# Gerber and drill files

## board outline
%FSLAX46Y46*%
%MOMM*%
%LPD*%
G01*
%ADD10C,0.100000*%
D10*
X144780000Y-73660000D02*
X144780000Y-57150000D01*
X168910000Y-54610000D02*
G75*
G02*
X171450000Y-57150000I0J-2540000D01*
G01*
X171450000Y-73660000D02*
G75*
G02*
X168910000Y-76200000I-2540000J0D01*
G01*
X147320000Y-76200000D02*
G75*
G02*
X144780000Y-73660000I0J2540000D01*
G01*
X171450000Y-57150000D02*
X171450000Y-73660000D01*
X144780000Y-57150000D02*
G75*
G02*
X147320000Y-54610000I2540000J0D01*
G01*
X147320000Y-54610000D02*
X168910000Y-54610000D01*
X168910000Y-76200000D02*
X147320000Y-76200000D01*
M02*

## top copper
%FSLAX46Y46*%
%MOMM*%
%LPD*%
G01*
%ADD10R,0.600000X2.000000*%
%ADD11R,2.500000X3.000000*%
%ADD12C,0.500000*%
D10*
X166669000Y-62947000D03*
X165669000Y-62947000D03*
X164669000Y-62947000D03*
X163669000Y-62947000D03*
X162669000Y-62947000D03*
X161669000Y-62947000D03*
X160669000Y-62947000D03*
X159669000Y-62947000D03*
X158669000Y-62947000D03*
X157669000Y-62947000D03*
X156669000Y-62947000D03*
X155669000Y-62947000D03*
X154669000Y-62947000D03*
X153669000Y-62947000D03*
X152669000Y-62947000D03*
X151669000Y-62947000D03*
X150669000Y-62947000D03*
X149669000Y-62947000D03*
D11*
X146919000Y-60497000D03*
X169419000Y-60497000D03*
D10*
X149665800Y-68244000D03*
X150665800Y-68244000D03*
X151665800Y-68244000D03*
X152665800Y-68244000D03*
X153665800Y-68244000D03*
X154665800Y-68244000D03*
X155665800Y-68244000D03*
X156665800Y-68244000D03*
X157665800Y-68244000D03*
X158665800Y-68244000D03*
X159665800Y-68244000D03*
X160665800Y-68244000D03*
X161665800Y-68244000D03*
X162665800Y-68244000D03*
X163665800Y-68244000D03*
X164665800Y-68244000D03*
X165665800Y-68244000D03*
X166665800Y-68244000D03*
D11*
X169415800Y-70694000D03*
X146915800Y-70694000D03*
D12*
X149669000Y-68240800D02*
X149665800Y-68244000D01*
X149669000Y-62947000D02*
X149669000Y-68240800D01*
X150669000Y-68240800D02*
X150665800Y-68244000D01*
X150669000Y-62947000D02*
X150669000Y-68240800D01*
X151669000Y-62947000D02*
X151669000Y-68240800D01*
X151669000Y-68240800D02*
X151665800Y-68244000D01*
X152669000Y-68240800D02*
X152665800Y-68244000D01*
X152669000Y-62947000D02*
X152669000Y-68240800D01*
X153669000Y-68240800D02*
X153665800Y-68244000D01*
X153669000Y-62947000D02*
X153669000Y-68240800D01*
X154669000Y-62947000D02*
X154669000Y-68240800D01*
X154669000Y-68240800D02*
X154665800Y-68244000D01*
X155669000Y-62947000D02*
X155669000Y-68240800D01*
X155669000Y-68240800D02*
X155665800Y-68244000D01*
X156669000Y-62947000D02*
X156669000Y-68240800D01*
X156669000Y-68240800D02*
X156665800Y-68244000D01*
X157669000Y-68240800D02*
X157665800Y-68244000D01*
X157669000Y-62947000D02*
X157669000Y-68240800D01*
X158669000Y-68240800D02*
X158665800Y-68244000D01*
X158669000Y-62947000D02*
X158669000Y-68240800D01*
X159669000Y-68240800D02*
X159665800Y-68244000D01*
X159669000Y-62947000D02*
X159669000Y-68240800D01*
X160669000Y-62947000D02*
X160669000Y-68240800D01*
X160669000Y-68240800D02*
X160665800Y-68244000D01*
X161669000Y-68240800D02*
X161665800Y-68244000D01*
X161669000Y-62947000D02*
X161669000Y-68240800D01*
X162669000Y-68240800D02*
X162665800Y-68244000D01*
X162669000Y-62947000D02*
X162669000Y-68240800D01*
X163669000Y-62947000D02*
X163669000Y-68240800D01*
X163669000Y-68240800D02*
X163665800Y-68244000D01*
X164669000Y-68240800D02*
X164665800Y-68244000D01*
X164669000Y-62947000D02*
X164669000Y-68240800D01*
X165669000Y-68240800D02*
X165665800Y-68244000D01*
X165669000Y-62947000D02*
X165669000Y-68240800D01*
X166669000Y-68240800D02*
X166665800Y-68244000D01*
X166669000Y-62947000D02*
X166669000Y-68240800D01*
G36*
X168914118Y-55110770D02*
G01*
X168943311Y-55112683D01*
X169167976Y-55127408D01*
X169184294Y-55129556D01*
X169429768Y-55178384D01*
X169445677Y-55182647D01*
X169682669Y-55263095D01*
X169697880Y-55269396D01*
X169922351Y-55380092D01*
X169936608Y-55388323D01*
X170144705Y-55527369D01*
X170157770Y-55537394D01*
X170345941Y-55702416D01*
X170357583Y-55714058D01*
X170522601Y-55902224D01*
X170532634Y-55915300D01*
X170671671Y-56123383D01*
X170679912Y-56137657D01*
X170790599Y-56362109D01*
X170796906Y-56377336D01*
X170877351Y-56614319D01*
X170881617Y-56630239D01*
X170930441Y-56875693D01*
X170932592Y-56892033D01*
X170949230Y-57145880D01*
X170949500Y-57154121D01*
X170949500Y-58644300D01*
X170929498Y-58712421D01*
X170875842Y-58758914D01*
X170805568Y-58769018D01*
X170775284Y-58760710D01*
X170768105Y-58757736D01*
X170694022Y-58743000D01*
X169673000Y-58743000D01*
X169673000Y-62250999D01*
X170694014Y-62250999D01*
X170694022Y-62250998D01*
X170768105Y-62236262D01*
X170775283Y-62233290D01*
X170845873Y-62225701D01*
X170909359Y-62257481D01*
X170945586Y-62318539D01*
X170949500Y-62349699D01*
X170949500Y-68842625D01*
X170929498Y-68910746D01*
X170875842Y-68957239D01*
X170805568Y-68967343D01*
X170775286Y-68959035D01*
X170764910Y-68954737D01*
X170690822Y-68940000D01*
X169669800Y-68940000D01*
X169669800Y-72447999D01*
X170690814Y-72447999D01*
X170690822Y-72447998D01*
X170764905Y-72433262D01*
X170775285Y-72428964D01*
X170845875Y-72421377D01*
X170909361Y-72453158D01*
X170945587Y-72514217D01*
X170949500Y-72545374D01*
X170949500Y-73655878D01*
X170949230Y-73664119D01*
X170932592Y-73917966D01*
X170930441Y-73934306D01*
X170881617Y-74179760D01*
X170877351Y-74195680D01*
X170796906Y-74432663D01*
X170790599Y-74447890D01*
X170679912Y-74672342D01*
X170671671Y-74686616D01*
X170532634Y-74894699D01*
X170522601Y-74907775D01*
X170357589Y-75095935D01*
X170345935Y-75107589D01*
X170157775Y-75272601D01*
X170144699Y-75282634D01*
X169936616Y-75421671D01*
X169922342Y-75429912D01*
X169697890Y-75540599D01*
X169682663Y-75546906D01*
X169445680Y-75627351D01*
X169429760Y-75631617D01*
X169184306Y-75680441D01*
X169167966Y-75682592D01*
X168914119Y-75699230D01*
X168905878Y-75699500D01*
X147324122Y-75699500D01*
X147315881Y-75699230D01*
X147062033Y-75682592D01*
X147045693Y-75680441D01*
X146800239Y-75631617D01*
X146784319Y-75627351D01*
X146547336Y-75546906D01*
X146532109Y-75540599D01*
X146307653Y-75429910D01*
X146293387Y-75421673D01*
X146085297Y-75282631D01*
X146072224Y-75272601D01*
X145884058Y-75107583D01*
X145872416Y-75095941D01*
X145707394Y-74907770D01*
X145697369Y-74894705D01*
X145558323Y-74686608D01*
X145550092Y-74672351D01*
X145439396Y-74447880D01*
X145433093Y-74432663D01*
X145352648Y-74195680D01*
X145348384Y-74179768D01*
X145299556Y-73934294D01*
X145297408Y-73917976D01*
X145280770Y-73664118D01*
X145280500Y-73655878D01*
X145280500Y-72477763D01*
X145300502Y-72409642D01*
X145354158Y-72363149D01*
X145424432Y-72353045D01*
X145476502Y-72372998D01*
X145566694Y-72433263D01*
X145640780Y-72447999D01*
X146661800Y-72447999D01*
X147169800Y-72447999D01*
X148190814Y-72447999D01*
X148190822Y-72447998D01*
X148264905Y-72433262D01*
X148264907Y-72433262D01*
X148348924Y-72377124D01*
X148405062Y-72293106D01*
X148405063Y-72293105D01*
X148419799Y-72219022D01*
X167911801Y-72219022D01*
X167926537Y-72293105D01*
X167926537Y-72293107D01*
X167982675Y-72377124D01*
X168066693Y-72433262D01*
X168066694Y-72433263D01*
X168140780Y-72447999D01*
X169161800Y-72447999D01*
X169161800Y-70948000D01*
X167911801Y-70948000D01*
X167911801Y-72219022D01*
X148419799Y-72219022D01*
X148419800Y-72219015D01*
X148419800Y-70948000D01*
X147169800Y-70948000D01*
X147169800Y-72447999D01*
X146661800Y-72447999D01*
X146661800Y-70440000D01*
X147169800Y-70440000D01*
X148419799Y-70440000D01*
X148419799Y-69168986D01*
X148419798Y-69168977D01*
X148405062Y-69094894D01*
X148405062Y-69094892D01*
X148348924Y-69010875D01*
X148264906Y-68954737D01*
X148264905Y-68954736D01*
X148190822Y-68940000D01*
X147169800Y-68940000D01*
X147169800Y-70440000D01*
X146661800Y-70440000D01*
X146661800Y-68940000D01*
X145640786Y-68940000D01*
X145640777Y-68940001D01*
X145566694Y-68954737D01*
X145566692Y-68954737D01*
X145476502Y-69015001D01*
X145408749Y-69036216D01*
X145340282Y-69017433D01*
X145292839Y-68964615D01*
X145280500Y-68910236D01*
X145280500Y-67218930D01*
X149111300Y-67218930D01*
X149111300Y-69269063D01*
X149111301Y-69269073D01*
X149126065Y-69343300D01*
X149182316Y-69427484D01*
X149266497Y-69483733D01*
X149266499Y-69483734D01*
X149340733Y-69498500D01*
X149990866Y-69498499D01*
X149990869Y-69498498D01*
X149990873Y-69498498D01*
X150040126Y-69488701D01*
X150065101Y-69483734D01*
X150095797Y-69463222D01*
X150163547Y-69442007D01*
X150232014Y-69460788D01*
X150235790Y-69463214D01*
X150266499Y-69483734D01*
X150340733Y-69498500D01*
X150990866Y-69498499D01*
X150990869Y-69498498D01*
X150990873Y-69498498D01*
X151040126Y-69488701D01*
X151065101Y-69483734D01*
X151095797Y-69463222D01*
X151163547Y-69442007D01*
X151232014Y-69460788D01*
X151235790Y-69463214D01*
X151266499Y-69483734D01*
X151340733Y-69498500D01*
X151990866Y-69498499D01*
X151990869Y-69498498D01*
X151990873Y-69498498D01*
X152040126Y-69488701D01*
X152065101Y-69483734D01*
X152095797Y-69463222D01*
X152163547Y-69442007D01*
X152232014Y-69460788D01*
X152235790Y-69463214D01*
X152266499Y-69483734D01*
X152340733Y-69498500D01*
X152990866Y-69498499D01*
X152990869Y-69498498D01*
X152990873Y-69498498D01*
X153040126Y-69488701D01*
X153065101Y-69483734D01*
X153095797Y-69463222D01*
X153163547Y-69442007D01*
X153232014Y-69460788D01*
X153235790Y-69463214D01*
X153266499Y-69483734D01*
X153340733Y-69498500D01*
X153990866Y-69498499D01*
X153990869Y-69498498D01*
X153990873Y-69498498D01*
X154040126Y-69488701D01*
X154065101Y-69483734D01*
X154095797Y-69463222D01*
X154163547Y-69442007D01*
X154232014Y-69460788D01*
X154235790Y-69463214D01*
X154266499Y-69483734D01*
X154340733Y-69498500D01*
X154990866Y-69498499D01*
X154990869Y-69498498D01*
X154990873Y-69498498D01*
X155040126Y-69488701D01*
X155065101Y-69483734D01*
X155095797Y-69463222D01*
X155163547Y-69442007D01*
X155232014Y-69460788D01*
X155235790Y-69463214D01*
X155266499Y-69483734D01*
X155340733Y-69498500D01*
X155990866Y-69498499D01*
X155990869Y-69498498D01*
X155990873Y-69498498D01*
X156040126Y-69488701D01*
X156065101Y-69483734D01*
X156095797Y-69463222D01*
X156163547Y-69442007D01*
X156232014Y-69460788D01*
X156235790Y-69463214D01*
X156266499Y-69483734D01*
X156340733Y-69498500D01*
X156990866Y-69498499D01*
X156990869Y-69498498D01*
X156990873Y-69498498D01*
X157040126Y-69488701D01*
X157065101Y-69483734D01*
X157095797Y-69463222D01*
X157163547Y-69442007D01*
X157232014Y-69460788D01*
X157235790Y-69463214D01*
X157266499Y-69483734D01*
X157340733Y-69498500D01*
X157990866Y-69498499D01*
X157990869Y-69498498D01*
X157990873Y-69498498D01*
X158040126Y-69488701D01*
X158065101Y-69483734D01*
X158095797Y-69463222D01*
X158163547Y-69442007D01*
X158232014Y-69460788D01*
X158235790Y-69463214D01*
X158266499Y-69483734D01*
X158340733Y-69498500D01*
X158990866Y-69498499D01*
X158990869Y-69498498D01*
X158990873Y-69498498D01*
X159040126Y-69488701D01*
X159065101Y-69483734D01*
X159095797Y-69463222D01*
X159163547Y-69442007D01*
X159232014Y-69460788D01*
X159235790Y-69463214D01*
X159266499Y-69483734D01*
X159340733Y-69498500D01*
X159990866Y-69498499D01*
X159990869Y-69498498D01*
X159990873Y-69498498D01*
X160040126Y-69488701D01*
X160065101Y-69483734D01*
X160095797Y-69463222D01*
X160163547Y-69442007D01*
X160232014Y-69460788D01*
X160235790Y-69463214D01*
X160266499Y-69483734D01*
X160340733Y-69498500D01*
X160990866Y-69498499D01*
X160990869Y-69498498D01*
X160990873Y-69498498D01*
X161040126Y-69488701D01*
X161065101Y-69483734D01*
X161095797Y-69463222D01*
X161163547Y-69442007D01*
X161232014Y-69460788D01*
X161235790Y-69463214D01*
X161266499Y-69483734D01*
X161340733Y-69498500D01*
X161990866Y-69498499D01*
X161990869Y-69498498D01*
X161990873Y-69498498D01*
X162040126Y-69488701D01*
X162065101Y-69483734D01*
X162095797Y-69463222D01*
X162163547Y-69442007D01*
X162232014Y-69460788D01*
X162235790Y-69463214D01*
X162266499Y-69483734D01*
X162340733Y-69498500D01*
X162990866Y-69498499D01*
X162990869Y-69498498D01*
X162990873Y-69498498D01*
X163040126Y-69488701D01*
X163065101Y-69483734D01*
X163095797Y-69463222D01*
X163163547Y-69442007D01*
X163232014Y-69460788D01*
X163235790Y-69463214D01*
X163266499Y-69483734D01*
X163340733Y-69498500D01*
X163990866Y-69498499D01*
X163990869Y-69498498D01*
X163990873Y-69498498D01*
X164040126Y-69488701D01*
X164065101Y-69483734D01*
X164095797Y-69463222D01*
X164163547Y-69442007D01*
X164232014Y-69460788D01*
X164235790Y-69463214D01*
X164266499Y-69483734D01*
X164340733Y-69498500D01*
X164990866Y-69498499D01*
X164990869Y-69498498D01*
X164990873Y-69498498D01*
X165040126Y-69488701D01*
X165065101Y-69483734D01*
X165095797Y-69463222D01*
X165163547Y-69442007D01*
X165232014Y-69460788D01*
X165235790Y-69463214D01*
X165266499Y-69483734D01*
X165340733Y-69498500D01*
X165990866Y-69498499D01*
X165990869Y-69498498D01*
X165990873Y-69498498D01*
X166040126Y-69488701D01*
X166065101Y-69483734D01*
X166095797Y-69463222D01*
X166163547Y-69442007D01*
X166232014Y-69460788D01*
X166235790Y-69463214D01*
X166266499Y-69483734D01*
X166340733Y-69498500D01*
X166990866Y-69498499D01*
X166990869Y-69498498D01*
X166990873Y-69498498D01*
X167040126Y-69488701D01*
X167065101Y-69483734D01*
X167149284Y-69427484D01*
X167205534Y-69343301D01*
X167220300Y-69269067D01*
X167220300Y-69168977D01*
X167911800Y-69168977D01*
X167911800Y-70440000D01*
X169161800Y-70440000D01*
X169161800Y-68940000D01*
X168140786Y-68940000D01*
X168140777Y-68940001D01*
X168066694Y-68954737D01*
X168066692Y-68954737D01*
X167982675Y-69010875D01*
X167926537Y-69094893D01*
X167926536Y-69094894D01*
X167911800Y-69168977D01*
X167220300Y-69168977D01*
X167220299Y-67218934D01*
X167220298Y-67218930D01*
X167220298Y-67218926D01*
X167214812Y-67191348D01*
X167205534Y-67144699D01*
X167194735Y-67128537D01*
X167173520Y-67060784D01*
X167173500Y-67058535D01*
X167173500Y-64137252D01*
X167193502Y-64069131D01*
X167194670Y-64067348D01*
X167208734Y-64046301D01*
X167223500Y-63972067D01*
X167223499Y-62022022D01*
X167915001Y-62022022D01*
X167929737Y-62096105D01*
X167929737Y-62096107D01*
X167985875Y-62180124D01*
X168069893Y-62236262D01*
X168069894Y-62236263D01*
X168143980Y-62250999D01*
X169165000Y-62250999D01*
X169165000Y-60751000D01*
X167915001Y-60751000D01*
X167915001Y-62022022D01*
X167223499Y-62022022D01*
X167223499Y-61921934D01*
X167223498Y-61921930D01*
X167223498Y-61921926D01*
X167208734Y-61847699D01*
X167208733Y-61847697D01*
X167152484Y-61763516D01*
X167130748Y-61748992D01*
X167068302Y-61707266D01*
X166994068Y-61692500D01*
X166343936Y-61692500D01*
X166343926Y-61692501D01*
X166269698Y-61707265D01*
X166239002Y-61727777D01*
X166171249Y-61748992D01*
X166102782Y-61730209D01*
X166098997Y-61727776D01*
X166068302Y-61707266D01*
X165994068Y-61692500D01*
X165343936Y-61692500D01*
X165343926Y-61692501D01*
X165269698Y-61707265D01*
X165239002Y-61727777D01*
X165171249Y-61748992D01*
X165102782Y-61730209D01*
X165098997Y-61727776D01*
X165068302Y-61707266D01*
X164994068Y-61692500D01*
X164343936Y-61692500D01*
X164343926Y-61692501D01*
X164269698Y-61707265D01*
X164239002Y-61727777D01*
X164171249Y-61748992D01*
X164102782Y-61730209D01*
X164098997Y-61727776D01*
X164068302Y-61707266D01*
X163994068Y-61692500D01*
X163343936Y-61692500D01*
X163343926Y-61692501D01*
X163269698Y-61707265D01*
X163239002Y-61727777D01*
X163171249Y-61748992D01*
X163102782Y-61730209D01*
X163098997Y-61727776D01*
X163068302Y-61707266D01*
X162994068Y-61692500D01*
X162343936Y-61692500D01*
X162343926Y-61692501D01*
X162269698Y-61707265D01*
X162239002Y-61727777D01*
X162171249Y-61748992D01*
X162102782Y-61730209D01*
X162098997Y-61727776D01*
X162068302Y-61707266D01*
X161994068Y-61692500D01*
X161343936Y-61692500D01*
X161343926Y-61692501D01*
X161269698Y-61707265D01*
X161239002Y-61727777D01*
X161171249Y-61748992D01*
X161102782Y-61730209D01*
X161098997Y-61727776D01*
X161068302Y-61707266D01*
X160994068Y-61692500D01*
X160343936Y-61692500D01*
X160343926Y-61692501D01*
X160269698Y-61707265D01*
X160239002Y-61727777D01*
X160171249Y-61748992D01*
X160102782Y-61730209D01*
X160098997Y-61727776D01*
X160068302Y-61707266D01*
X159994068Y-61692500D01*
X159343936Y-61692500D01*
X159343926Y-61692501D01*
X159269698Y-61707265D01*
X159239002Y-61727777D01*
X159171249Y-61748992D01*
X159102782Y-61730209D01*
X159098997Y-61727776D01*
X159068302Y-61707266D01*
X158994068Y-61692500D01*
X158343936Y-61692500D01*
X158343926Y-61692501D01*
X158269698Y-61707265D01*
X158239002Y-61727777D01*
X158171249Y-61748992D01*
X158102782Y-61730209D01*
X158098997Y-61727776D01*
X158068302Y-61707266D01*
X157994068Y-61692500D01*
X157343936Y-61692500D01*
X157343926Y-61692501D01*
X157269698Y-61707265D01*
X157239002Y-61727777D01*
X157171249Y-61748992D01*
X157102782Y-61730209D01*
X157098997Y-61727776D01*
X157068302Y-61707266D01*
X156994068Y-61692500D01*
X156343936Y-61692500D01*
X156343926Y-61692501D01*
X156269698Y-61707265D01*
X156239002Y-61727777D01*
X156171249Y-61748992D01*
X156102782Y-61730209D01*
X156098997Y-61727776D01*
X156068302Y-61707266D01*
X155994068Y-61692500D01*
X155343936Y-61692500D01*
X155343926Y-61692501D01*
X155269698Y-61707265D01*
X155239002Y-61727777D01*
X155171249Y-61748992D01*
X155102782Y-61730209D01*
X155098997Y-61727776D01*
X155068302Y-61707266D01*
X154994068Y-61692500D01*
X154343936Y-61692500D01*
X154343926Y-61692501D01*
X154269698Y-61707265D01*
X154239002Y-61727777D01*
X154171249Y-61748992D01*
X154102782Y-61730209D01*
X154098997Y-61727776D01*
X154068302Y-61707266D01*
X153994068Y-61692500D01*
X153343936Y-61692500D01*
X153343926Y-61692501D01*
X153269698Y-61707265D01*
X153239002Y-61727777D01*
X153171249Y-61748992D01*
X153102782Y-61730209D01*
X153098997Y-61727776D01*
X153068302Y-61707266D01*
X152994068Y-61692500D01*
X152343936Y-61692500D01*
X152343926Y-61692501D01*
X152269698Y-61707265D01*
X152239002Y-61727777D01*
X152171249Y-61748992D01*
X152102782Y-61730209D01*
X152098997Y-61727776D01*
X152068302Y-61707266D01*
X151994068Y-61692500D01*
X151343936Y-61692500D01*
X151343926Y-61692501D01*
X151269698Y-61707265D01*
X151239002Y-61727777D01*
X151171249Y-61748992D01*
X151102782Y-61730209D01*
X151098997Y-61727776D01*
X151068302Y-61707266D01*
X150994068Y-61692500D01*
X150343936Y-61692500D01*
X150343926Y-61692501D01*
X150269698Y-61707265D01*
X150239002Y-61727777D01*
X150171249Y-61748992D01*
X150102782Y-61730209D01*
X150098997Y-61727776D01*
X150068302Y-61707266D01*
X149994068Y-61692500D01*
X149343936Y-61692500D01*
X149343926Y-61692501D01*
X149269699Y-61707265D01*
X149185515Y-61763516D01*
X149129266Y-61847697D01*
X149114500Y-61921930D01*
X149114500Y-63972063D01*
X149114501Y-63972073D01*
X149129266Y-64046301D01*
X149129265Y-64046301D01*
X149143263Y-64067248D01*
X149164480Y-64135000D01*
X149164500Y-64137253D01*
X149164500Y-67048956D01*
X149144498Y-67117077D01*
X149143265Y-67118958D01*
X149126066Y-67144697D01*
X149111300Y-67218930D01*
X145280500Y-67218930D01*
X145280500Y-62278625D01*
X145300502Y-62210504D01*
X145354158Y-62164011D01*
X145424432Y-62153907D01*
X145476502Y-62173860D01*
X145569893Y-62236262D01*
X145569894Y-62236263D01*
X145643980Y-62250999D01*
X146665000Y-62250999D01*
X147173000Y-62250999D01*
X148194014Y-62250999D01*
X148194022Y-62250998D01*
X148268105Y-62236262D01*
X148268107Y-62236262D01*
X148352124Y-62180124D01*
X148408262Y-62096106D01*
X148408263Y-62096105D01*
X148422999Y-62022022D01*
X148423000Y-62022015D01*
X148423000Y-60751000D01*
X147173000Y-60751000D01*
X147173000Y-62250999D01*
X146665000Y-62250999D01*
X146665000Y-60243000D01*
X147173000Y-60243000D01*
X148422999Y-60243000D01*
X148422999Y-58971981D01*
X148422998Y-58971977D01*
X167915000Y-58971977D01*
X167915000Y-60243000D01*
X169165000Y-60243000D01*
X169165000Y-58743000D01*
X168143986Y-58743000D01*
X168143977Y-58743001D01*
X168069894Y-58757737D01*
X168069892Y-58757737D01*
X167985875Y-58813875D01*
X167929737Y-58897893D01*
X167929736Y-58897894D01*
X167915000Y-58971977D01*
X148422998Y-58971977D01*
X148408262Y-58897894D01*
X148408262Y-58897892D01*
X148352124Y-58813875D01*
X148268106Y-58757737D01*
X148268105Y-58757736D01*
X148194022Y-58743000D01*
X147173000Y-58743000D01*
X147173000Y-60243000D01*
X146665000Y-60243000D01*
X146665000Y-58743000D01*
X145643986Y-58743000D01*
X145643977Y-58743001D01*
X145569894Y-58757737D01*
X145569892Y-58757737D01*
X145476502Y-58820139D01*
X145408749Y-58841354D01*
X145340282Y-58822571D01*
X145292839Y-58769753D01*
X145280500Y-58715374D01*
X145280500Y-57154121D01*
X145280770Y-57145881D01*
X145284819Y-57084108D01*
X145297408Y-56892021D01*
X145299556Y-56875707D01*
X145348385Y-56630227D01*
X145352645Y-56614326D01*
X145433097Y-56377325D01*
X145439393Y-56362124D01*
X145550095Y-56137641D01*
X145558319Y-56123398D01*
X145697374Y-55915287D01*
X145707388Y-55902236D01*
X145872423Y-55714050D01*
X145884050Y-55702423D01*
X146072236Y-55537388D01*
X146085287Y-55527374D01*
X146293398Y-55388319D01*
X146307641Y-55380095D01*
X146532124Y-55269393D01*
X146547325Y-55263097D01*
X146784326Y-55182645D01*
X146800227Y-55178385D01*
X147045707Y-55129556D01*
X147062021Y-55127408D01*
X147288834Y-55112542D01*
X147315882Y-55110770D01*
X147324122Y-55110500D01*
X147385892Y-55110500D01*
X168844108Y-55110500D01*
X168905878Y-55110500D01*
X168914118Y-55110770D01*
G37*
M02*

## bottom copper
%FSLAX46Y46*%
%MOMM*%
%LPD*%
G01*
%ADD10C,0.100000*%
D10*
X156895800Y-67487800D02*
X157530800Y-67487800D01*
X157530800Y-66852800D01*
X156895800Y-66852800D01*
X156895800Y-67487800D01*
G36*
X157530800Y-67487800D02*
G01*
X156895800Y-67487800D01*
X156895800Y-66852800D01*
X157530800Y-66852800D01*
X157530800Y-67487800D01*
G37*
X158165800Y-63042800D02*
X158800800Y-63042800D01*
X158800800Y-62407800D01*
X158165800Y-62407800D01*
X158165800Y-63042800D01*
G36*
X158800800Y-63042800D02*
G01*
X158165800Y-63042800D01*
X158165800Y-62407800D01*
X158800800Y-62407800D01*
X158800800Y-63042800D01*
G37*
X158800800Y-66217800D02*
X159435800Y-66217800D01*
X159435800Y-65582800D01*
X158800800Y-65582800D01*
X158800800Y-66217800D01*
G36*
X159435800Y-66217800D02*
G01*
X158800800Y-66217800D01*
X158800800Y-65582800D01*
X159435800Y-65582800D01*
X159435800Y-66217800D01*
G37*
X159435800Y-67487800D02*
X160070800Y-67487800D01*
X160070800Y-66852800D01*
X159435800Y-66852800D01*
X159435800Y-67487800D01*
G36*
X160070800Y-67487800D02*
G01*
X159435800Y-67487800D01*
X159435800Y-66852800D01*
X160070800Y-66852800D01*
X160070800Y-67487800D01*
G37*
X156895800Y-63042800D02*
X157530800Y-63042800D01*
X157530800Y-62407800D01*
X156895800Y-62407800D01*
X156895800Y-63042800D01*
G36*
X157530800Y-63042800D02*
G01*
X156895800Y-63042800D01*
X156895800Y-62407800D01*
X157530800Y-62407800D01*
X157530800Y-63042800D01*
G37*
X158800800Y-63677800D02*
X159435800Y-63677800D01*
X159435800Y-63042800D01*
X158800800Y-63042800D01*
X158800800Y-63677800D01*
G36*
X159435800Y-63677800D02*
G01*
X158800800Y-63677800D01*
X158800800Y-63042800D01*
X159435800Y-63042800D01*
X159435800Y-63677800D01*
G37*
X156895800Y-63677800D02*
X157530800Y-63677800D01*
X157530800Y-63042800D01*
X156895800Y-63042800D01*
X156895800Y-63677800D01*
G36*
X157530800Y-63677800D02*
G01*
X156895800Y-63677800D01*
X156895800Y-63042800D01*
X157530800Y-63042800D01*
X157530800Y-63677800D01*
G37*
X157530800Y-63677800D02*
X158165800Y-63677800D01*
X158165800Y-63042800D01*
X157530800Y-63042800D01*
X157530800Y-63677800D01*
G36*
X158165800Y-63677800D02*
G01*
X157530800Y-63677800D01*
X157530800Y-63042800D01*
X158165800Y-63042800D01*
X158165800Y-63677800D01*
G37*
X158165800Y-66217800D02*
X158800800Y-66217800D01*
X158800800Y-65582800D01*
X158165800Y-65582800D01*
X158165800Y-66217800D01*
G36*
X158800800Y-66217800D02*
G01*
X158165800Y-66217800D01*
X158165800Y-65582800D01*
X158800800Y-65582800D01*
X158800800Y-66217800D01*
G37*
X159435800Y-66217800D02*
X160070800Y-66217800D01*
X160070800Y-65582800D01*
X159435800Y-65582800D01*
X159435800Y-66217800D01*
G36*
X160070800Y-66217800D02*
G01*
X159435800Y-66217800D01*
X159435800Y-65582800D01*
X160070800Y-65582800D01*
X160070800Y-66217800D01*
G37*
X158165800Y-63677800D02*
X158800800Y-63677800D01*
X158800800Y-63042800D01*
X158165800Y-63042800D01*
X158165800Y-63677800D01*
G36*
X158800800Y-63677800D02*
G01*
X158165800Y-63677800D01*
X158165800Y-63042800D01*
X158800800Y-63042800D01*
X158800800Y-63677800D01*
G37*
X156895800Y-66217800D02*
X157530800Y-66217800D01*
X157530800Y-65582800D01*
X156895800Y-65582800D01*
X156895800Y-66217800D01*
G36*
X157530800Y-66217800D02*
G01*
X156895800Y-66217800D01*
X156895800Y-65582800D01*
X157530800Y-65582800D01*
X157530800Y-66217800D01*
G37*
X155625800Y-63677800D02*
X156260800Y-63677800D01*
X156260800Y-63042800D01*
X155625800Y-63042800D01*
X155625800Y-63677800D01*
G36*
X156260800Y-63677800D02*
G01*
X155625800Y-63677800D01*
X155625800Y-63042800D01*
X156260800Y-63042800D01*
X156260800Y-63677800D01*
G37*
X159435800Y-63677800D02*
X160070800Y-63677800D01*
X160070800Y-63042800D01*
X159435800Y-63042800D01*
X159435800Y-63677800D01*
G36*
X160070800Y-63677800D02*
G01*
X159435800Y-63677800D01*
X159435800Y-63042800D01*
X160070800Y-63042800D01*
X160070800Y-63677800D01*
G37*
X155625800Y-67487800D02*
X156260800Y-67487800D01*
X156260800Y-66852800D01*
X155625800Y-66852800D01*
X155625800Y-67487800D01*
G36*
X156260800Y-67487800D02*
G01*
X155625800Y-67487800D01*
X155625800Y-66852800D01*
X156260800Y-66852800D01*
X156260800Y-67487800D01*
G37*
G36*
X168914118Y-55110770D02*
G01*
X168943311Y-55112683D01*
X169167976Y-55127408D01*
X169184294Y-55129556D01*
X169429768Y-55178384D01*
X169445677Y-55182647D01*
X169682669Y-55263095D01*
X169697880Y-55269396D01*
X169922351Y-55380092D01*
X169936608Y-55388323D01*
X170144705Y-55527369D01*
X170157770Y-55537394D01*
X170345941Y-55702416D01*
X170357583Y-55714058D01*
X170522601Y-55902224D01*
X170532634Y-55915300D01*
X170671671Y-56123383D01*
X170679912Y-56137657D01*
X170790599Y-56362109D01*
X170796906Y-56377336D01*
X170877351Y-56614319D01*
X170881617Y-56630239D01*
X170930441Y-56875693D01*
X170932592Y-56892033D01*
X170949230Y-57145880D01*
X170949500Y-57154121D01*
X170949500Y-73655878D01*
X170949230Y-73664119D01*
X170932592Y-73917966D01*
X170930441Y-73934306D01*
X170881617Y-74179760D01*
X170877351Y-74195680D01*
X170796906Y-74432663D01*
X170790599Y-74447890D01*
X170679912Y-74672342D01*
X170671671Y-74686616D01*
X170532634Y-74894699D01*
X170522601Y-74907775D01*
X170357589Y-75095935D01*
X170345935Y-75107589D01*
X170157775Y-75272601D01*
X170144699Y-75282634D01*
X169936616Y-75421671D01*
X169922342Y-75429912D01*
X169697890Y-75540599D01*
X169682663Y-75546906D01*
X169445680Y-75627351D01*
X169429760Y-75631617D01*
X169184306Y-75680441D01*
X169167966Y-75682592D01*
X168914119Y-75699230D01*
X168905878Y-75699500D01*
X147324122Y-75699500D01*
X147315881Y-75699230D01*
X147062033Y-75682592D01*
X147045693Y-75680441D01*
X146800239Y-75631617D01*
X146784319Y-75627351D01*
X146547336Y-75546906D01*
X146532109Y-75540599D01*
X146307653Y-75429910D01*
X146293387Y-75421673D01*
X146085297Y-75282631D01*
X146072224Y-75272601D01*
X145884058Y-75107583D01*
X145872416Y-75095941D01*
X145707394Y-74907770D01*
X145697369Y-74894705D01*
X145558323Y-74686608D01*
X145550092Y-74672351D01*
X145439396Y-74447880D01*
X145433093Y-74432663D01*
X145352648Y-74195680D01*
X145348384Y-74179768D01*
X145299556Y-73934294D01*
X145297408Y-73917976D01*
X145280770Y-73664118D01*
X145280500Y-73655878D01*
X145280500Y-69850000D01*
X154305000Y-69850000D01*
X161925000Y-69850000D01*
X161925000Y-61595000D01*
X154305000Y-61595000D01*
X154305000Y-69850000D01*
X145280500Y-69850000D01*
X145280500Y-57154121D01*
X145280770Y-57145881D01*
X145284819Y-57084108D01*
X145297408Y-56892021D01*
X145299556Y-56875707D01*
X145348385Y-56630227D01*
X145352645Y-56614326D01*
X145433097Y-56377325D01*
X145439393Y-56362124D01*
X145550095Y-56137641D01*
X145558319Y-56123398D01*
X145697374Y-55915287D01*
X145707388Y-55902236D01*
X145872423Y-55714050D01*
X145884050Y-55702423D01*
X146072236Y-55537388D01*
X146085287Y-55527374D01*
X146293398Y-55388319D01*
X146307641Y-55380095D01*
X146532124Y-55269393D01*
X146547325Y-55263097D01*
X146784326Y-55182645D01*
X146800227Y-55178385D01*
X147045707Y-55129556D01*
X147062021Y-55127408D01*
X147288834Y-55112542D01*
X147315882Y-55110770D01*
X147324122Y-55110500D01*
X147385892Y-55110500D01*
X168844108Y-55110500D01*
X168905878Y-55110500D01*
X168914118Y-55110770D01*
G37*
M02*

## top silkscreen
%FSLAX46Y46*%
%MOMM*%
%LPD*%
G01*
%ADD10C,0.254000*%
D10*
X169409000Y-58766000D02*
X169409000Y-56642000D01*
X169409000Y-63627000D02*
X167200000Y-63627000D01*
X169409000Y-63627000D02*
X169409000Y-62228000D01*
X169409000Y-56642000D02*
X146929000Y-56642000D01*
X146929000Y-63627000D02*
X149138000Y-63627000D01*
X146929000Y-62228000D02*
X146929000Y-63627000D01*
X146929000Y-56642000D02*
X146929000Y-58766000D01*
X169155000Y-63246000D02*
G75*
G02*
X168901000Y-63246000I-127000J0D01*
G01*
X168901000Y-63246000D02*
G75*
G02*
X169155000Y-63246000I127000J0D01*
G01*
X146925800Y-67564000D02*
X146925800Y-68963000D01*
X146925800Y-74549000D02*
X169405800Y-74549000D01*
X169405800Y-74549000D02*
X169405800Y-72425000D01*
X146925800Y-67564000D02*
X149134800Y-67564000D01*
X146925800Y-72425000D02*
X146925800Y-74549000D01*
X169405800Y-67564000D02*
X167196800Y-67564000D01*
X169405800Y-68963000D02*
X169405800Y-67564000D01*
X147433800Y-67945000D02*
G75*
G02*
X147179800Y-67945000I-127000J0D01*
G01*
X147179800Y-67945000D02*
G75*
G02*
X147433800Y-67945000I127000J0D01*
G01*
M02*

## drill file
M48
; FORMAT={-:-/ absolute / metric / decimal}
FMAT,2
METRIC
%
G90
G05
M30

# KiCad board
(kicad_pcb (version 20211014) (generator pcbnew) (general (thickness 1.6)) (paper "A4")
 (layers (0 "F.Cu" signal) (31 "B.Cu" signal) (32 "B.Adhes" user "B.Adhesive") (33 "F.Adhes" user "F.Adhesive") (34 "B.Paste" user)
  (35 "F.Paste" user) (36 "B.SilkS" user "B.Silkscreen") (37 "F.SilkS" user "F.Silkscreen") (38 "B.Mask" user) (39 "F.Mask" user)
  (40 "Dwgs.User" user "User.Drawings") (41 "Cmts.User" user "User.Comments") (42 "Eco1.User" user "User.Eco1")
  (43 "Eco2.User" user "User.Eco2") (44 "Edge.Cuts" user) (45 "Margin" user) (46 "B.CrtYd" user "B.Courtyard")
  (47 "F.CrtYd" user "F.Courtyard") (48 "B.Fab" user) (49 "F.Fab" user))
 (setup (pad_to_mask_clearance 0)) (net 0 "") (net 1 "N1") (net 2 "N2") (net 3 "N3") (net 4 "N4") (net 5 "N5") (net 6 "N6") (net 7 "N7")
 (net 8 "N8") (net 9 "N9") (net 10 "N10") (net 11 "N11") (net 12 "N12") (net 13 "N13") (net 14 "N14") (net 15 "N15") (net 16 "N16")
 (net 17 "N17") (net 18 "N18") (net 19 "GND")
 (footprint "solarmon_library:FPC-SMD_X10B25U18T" (layer "F.Cu") (at 158.169 62.992)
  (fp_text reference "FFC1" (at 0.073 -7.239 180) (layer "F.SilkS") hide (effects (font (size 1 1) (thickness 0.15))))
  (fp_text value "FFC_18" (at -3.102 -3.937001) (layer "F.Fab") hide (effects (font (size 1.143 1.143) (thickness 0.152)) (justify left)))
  (fp_line (start 11.24 -4.226) (end 11.24 -6.35) (layer "F.SilkS") (width 0.254))
  (fp_line (start 11.24 0.635) (end 9.031 0.635) (layer "F.SilkS") (width 0.254))
  (fp_line (start 11.24 0.635) (end 11.24 -0.764) (layer "F.SilkS") (width 0.254))
  (fp_line (start 11.24 -6.35) (end -11.24 -6.35) (layer "F.SilkS") (width 0.254))
  (fp_line (start -11.24 0.635) (end -9.031 0.635) (layer "F.SilkS") (width 0.254))
  (fp_line (start -11.24 -0.764) (end -11.24 0.635) (layer "F.SilkS") (width 0.254))
  (fp_line (start -11.24 -6.35) (end -11.24 -4.226) (layer "F.SilkS") (width 0.254))
  (fp_circle (center 10.859 0.254) (end 10.732 0.254) (layer "F.SilkS") (width 0.254) (fill none))
  (pad "1" smd rect locked (at 8.5 -0.045 180) (size 0.6 2) (layers "F.Cu" "F.Paste" "F.Mask") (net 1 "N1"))
  (pad "2" smd rect locked (at 7.5 -0.045 180) (size 0.6 2) (layers "F.Cu" "F.Paste" "F.Mask") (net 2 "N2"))
  (pad "3" smd rect locked (at 6.5 -0.045 180) (size 0.6 2) (layers "F.Cu" "F.Paste" "F.Mask") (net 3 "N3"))
  (pad "4" smd rect locked (at 5.5 -0.045 180) (size 0.6 2) (layers "F.Cu" "F.Paste" "F.Mask") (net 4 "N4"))
  (pad "5" smd rect locked (at 4.5 -0.045 180) (size 0.6 2) (layers "F.Cu" "F.Paste" "F.Mask") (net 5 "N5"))
  (pad "6" smd rect locked (at 3.5 -0.045 180) (size 0.6 2) (layers "F.Cu" "F.Paste" "F.Mask") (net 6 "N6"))
  (pad "7" smd rect locked (at 2.5 -0.045 180) (size 0.6 2) (layers "F.Cu" "F.Paste" "F.Mask") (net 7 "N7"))
  (pad "8" smd rect locked (at 1.5 -0.045 180) (size 0.6 2) (layers "F.Cu" "F.Paste" "F.Mask") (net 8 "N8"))
  (pad "9" smd rect locked (at 0.5 -0.045 180) (size 0.6 2) (layers "F.Cu" "F.Paste" "F.Mask") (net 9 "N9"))
  (pad "10" smd rect locked (at -0.5 -0.045 180) (size 0.6 2) (layers "F.Cu" "F.Paste" "F.Mask") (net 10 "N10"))
  (pad "11" smd rect locked (at -1.5 -0.045 180) (size 0.6 2) (layers "F.Cu" "F.Paste" "F.Mask") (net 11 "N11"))
  (pad "12" smd rect locked (at -2.5 -0.045 180) (size 0.6 2) (layers "F.Cu" "F.Paste" "F.Mask") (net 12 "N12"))
  (pad "13" smd rect locked (at -3.5 -0.045 180) (size 0.6 2) (layers "F.Cu" "F.Paste" "F.Mask") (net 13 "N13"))
  (pad "14" smd rect locked (at -4.5 -0.045 180) (size 0.6 2) (layers "F.Cu" "F.Paste" "F.Mask") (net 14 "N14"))
  (pad "15" smd rect locked (at -5.5 -0.045 180) (size 0.6 2) (layers "F.Cu" "F.Paste" "F.Mask") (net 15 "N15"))
  (pad "16" smd rect locked (at -6.5 -0.045 180) (size 0.6 2) (layers "F.Cu" "F.Paste" "F.Mask") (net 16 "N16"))
  (pad "17" smd rect locked (at -7.5 -0.045 180) (size 0.6 2) (layers "F.Cu" "F.Paste" "F.Mask") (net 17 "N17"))
  (pad "18" smd rect locked (at -8.5 -0.045 180) (size 0.6 2) (layers "F.Cu" "F.Paste" "F.Mask") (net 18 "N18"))
  (pad "MP" smd rect locked (at -11.25 -2.495 180) (size 2.5 3) (layers "F.Cu" "F.Paste" "F.Mask") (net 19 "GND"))
  (pad "MP" smd rect locked (at 11.25 -2.495 180) (size 2.5 3) (layers "F.Cu" "F.Paste" "F.Mask") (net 19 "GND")))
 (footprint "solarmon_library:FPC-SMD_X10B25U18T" (layer "F.Cu") (at 158.1658 68.199 180)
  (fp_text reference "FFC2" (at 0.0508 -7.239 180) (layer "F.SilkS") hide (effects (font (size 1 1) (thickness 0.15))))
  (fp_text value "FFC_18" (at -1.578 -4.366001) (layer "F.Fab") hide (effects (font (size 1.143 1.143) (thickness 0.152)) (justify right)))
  (fp_line (start 11.24 0.635) (end 11.24 -0.764) (layer "F.SilkS") (width 0.254))
  (fp_line (start 11.24 -6.35) (end -11.24 -6.35) (layer "F.SilkS") (width 0.254))
  (fp_line (start -11.24 -6.35) (end -11.24 -4.226) (layer "F.SilkS") (width 0.254))
  (fp_line (start 11.24 0.635) (end 9.031 0.635) (layer "F.SilkS") (width 0.254))
  (fp_line (start 11.24 -4.226) (end 11.24 -6.35) (layer "F.SilkS") (width 0.254))
  (fp_line (start -11.24 0.635) (end -9.031 0.635) (layer "F.SilkS") (width 0.254))
  (fp_line (start -11.24 -0.764) (end -11.24 0.635) (layer "F.SilkS") (width 0.254))
  (fp_circle (center 10.859 0.254) (end 10.732 0.254) (layer "F.SilkS") (width 0.254) (fill none))
  (pad "1" smd rect locked (at 8.5 -0.045) (size 0.6 2) (layers "F.Cu" "F.Paste" "F.Mask") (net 18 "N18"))
  (pad "2" smd rect locked (at 7.5 -0.045) (size 0.6 2) (layers "F.Cu" "F.Paste" "F.Mask") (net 17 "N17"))
  (pad "3" smd rect locked (at 6.5 -0.045) (size 0.6 2) (layers "F.Cu" "F.Paste" "F.Mask") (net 16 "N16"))
  (pad "4" smd rect locked (at 5.5 -0.045) (size 0.6 2) (layers "F.Cu" "F.Paste" "F.Mask") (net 15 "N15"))
  (pad "5" smd rect locked (at 4.5 -0.045) (size 0.6 2) (layers "F.Cu" "F.Paste" "F.Mask") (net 14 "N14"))
  (pad "6" smd rect locked (at 3.5 -0.045) (size 0.6 2) (layers "F.Cu" "F.Paste" "F.Mask") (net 13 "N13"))
  (pad "7" smd rect locked (at 2.5 -0.045) (size 0.6 2) (layers "F.Cu" "F.Paste" "F.Mask") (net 12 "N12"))
  (pad "8" smd rect locked (at 1.5 -0.045) (size 0.6 2) (layers "F.Cu" "F.Paste" "F.Mask") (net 11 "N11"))
  (pad "9" smd rect locked (at 0.5 -0.045) (size 0.6 2) (layers "F.Cu" "F.Paste" "F.Mask") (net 10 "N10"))
  (pad "10" smd rect locked (at -0.5 -0.045) (size 0.6 2) (layers "F.Cu" "F.Paste" "F.Mask") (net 9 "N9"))
  (pad "11" smd rect locked (at -1.5 -0.045) (size 0.6 2) (layers "F.Cu" "F.Paste" "F.Mask") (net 8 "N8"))
  (pad "12" smd rect locked (at -2.5 -0.045) (size 0.6 2) (layers "F.Cu" "F.Paste" "F.Mask") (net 7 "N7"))
  (pad "13" smd rect locked (at -3.5 -0.045) (size 0.6 2) (layers "F.Cu" "F.Paste" "F.Mask") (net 6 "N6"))
  (pad "14" smd rect locked (at -4.5 -0.045) (size 0.6 2) (layers "F.Cu" "F.Paste" "F.Mask") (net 5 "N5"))
  (pad "15" smd rect locked (at -5.5 -0.045) (size 0.6 2) (layers "F.Cu" "F.Paste" "F.Mask") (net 4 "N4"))
  (pad "16" smd rect locked (at -6.5 -0.045) (size 0.6 2) (layers "F.Cu" "F.Paste" "F.Mask") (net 3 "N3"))
  (pad "17" smd rect locked (at -7.5 -0.045) (size 0.6 2) (layers "F.Cu" "F.Paste" "F.Mask") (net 2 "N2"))
  (pad "18" smd rect locked (at -8.5 -0.045) (size 0.6 2) (layers "F.Cu" "F.Paste" "F.Mask") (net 1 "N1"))
  (pad "MP" smd rect locked (at -11.25 -2.495) (size 2.5 3) (layers "F.Cu" "F.Paste" "F.Mask") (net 19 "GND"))
  (pad "MP" smd rect locked (at 11.25 -2.495) (size 2.5 3) (layers "F.Cu" "F.Paste" "F.Mask") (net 19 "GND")))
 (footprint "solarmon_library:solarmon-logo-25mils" (layer "B.Cu") (at 158.1658 65.5828 180)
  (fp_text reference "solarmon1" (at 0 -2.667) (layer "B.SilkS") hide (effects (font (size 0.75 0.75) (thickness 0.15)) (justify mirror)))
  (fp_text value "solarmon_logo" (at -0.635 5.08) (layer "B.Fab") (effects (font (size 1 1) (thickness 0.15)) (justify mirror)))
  (fp_poly (pts (xy 1.27 -1.905) (xy 0.635 -1.905) (xy 0.635 -1.27) (xy 1.27 -1.27)) (layer "B.Cu") (width 0.1) (fill solid))
  (fp_poly (pts (xy 0 2.54) (xy -0.635 2.54) (xy -0.635 3.175) (xy 0 3.175)) (layer "B.Cu") (width 0.1) (fill solid))
  (fp_poly (pts (xy -0.635 -0.635) (xy -1.27 -0.635) (xy -1.27 0) (xy -0.635 0)) (layer "B.Cu") (width 0.1) (fill solid))
  (fp_poly (pts (xy -1.27 -1.905) (xy -1.905 -1.905) (xy -1.905 -1.27) (xy -1.27 -1.27)) (layer "B.Cu") (width 0.1) (fill solid))
  (fp_poly (pts (xy 1.27 2.54) (xy 0.635 2.54) (xy 0.635 3.175) (xy 1.27 3.175)) (layer "B.Cu") (width 0.1) (fill solid))
  (fp_poly (pts (xy -0.635 1.905) (xy -1.27 1.905) (xy -1.27 2.54) (xy -0.635 2.54)) (layer "B.Cu") (width 0.1) (fill solid))
  (fp_poly (pts (xy 1.27 1.905) (xy 0.635 1.905) (xy 0.635 2.54) (xy 1.27 2.54)) (layer "B.Cu") (width 0.1) (fill solid))
  (fp_poly (pts (xy 0.635 1.905) (xy 0 1.905) (xy 0 2.54) (xy 0.635 2.54)) (layer "B.Cu") (width 0.1) (fill solid))
  (fp_poly (pts (xy 0 -0.635) (xy -0.635 -0.635) (xy -0.635 0) (xy 0 0)) (layer "B.Cu") (width 0.1) (fill solid))
  (fp_poly (pts (xy -1.27 -0.635) (xy -1.905 -0.635) (xy -1.905 0) (xy -1.27 0)) (layer "B.Cu") (width 0.1) (fill solid))
  (fp_poly (pts (xy 0 1.905) (xy -0.635 1.905) (xy -0.635 2.54) (xy 0 2.54)) (layer "B.Cu") (width 0.1) (fill solid))
  (fp_poly (pts (xy 1.27 -0.635) (xy 0.635 -0.635) (xy 0.635 0) (xy 1.27 0)) (layer "B.Cu") (width 0.1) (fill solid))
  (fp_poly (pts (xy 2.54 1.905) (xy 1.905 1.905) (xy 1.905 2.54) (xy 2.54 2.54)) (layer "B.Cu") (width 0.1) (fill solid))
  (fp_poly (pts (xy -1.27 1.905) (xy -1.905 1.905) (xy -1.905 2.54) (xy -1.27 2.54)) (layer "B.Cu") (width 0.1) (fill solid))
  (fp_poly (pts (xy 2.54 -1.905) (xy 1.905 -1.905) (xy 1.905 -1.27) (xy 2.54 -1.27)) (layer "B.Cu") (width 0.1) (fill solid)))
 (gr_line (start 144.78 73.66) (end 144.78 57.15) (layer "Edge.Cuts") (width 0.1))
 (gr_arc (start 168.91 54.61) (mid 170.706051 55.353949) (end 171.45 57.15) (layer "Edge.Cuts") (width 0.1))
 (gr_arc (start 171.45 73.66) (mid 170.706051 75.456051) (end 168.91 76.2) (layer "Edge.Cuts") (width 0.1))
 (gr_arc (start 147.32 76.2) (mid 145.523949 75.456051) (end 144.78 73.66) (layer "Edge.Cuts") (width 0.1))
 (gr_line (start 171.45 57.15) (end 171.45 73.66) (layer "Edge.Cuts") (width 0.1))
 (gr_arc (start 144.78 57.15) (mid 145.523949 55.353949) (end 147.32 54.61) (layer "Edge.Cuts") (width 0.1))
 (gr_line (start 147.32 54.61) (end 168.91 54.61) (layer "Edge.Cuts") (width 0.1))
 (gr_line (start 168.91 76.2) (end 147.32 76.2) (layer "Edge.Cuts") (width 0.1))
 (segment (start 149.669 68.2408) (end 149.6658 68.244) (width 0.5) (layer "F.Cu") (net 18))
 (segment (start 149.669 62.947) (end 149.669 68.2408) (width 0.5) (layer "F.Cu") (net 18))
 (segment (start 150.669 68.2408) (end 150.6658 68.244) (width 0.5) (layer "F.Cu") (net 17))
 (segment (start 150.669 62.947) (end 150.669 68.2408) (width 0.5) (layer "F.Cu") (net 17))
 (segment (start 151.669 62.947) (end 151.669 68.2408) (width 0.5) (layer "F.Cu") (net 16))
 (segment (start 151.669 68.2408) (end 151.6658 68.244) (width 0.5) (layer "F.Cu") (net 16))
 (segment (start 152.669 68.2408) (end 152.6658 68.244) (width 0.5) (layer "F.Cu") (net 15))
 (segment (start 152.669 62.947) (end 152.669 68.2408) (width 0.5) (layer "F.Cu") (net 15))
 (segment (start 153.669 68.2408) (end 153.6658 68.244) (width 0.5) (layer "F.Cu") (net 14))
 (segment (start 153.669 62.947) (end 153.669 68.2408) (width 0.5) (layer "F.Cu") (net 14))
 (segment (start 154.669 62.947) (end 154.669 68.2408) (width 0.5) (layer "F.Cu") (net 13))
 (segment (start 154.669 68.2408) (end 154.6658 68.244) (width 0.5) (layer "F.Cu") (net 13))
 (segment (start 155.669 62.947) (end 155.669 68.2408) (width 0.5) (layer "F.Cu") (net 12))
 (segment (start 155.669 68.2408) (end 155.6658 68.244) (width 0.5) (layer "F.Cu") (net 12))
 (segment (start 156.669 62.947) (end 156.669 68.2408) (width 0.5) (layer "F.Cu") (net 11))
 (segment (start 156.669 68.2408) (end 156.6658 68.244) (width 0.5) (layer "F.Cu") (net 11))
 (segment (start 157.669 68.2408) (end 157.6658 68.244) (width 0.5) (layer "F.Cu") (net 10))
 (segment (start 157.669 62.947) (end 157.669 68.2408) (width 0.5) (layer "F.Cu") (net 10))
 (segment (start 158.669 68.2408) (end 158.6658 68.244) (width 0.5) (layer "F.Cu") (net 9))
 (segment (start 158.669 62.947) (end 158.669 68.2408) (width 0.5) (layer "F.Cu") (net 9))
 (segment (start 159.669 68.2408) (end 159.6658 68.244) (width 0.5) (layer "F.Cu") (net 8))
 (segment (start 159.669 62.947) (end 159.669 68.2408) (width 0.5) (layer "F.Cu") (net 8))
 (segment (start 160.669 62.947) (end 160.669 68.2408) (width 0.5) (layer "F.Cu") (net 7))
 (segment (start 160.669 68.2408) (end 160.6658 68.244) (width 0.5) (layer "F.Cu") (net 7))
 (segment (start 161.669 68.2408) (end 161.6658 68.244) (width 0.5) (layer "F.Cu") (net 6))
 (segment (start 161.669 62.947) (end 161.669 68.2408) (width 0.5) (layer "F.Cu") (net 6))
 (segment (start 162.669 68.2408) (end 162.6658 68.244) (width 0.5) (layer "F.Cu") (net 5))
 (segment (start 162.669 62.947) (end 162.669 68.2408) (width 0.5) (layer "F.Cu") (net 5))
 (segment (start 163.669 62.947) (end 163.669 68.2408) (width 0.5) (layer "F.Cu") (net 4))
 (segment (start 163.669 68.2408) (end 163.6658 68.244) (width 0.5) (layer "F.Cu") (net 4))
 (segment (start 164.669 68.2408) (end 164.6658 68.244) (width 0.5) (layer "F.Cu") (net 3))
 (segment (start 164.669 62.947) (end 164.669 68.2408) (width 0.5) (layer "F.Cu") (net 3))
 (segment (start 165.669 68.2408) (end 165.6658 68.244) (width 0.5) (layer "F.Cu") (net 2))
 (segment (start 165.669 62.947) (end 165.669 68.2408) (width 0.5) (layer "F.Cu") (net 2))
 (segment (start 166.669 68.2408) (end 166.6658 68.244) (width 0.5) (layer "F.Cu") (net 1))
 (segment (start 166.669 62.947) (end 166.669 68.2408) (width 0.5) (layer "F.Cu") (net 1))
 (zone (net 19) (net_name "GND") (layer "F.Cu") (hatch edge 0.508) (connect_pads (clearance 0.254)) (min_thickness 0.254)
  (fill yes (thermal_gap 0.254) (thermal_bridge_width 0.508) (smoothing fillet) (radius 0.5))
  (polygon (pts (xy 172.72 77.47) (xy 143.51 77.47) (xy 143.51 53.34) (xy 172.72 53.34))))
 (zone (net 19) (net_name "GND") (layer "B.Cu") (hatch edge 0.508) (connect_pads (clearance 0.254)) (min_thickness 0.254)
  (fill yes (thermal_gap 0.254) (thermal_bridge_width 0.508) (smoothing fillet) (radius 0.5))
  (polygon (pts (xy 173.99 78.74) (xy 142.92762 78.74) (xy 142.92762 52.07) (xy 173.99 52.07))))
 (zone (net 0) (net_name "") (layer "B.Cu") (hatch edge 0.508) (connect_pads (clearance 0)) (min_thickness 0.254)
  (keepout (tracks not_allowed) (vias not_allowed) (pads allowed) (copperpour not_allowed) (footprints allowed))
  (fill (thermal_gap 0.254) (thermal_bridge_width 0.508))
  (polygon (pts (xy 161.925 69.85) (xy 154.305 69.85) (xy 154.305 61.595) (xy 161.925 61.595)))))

